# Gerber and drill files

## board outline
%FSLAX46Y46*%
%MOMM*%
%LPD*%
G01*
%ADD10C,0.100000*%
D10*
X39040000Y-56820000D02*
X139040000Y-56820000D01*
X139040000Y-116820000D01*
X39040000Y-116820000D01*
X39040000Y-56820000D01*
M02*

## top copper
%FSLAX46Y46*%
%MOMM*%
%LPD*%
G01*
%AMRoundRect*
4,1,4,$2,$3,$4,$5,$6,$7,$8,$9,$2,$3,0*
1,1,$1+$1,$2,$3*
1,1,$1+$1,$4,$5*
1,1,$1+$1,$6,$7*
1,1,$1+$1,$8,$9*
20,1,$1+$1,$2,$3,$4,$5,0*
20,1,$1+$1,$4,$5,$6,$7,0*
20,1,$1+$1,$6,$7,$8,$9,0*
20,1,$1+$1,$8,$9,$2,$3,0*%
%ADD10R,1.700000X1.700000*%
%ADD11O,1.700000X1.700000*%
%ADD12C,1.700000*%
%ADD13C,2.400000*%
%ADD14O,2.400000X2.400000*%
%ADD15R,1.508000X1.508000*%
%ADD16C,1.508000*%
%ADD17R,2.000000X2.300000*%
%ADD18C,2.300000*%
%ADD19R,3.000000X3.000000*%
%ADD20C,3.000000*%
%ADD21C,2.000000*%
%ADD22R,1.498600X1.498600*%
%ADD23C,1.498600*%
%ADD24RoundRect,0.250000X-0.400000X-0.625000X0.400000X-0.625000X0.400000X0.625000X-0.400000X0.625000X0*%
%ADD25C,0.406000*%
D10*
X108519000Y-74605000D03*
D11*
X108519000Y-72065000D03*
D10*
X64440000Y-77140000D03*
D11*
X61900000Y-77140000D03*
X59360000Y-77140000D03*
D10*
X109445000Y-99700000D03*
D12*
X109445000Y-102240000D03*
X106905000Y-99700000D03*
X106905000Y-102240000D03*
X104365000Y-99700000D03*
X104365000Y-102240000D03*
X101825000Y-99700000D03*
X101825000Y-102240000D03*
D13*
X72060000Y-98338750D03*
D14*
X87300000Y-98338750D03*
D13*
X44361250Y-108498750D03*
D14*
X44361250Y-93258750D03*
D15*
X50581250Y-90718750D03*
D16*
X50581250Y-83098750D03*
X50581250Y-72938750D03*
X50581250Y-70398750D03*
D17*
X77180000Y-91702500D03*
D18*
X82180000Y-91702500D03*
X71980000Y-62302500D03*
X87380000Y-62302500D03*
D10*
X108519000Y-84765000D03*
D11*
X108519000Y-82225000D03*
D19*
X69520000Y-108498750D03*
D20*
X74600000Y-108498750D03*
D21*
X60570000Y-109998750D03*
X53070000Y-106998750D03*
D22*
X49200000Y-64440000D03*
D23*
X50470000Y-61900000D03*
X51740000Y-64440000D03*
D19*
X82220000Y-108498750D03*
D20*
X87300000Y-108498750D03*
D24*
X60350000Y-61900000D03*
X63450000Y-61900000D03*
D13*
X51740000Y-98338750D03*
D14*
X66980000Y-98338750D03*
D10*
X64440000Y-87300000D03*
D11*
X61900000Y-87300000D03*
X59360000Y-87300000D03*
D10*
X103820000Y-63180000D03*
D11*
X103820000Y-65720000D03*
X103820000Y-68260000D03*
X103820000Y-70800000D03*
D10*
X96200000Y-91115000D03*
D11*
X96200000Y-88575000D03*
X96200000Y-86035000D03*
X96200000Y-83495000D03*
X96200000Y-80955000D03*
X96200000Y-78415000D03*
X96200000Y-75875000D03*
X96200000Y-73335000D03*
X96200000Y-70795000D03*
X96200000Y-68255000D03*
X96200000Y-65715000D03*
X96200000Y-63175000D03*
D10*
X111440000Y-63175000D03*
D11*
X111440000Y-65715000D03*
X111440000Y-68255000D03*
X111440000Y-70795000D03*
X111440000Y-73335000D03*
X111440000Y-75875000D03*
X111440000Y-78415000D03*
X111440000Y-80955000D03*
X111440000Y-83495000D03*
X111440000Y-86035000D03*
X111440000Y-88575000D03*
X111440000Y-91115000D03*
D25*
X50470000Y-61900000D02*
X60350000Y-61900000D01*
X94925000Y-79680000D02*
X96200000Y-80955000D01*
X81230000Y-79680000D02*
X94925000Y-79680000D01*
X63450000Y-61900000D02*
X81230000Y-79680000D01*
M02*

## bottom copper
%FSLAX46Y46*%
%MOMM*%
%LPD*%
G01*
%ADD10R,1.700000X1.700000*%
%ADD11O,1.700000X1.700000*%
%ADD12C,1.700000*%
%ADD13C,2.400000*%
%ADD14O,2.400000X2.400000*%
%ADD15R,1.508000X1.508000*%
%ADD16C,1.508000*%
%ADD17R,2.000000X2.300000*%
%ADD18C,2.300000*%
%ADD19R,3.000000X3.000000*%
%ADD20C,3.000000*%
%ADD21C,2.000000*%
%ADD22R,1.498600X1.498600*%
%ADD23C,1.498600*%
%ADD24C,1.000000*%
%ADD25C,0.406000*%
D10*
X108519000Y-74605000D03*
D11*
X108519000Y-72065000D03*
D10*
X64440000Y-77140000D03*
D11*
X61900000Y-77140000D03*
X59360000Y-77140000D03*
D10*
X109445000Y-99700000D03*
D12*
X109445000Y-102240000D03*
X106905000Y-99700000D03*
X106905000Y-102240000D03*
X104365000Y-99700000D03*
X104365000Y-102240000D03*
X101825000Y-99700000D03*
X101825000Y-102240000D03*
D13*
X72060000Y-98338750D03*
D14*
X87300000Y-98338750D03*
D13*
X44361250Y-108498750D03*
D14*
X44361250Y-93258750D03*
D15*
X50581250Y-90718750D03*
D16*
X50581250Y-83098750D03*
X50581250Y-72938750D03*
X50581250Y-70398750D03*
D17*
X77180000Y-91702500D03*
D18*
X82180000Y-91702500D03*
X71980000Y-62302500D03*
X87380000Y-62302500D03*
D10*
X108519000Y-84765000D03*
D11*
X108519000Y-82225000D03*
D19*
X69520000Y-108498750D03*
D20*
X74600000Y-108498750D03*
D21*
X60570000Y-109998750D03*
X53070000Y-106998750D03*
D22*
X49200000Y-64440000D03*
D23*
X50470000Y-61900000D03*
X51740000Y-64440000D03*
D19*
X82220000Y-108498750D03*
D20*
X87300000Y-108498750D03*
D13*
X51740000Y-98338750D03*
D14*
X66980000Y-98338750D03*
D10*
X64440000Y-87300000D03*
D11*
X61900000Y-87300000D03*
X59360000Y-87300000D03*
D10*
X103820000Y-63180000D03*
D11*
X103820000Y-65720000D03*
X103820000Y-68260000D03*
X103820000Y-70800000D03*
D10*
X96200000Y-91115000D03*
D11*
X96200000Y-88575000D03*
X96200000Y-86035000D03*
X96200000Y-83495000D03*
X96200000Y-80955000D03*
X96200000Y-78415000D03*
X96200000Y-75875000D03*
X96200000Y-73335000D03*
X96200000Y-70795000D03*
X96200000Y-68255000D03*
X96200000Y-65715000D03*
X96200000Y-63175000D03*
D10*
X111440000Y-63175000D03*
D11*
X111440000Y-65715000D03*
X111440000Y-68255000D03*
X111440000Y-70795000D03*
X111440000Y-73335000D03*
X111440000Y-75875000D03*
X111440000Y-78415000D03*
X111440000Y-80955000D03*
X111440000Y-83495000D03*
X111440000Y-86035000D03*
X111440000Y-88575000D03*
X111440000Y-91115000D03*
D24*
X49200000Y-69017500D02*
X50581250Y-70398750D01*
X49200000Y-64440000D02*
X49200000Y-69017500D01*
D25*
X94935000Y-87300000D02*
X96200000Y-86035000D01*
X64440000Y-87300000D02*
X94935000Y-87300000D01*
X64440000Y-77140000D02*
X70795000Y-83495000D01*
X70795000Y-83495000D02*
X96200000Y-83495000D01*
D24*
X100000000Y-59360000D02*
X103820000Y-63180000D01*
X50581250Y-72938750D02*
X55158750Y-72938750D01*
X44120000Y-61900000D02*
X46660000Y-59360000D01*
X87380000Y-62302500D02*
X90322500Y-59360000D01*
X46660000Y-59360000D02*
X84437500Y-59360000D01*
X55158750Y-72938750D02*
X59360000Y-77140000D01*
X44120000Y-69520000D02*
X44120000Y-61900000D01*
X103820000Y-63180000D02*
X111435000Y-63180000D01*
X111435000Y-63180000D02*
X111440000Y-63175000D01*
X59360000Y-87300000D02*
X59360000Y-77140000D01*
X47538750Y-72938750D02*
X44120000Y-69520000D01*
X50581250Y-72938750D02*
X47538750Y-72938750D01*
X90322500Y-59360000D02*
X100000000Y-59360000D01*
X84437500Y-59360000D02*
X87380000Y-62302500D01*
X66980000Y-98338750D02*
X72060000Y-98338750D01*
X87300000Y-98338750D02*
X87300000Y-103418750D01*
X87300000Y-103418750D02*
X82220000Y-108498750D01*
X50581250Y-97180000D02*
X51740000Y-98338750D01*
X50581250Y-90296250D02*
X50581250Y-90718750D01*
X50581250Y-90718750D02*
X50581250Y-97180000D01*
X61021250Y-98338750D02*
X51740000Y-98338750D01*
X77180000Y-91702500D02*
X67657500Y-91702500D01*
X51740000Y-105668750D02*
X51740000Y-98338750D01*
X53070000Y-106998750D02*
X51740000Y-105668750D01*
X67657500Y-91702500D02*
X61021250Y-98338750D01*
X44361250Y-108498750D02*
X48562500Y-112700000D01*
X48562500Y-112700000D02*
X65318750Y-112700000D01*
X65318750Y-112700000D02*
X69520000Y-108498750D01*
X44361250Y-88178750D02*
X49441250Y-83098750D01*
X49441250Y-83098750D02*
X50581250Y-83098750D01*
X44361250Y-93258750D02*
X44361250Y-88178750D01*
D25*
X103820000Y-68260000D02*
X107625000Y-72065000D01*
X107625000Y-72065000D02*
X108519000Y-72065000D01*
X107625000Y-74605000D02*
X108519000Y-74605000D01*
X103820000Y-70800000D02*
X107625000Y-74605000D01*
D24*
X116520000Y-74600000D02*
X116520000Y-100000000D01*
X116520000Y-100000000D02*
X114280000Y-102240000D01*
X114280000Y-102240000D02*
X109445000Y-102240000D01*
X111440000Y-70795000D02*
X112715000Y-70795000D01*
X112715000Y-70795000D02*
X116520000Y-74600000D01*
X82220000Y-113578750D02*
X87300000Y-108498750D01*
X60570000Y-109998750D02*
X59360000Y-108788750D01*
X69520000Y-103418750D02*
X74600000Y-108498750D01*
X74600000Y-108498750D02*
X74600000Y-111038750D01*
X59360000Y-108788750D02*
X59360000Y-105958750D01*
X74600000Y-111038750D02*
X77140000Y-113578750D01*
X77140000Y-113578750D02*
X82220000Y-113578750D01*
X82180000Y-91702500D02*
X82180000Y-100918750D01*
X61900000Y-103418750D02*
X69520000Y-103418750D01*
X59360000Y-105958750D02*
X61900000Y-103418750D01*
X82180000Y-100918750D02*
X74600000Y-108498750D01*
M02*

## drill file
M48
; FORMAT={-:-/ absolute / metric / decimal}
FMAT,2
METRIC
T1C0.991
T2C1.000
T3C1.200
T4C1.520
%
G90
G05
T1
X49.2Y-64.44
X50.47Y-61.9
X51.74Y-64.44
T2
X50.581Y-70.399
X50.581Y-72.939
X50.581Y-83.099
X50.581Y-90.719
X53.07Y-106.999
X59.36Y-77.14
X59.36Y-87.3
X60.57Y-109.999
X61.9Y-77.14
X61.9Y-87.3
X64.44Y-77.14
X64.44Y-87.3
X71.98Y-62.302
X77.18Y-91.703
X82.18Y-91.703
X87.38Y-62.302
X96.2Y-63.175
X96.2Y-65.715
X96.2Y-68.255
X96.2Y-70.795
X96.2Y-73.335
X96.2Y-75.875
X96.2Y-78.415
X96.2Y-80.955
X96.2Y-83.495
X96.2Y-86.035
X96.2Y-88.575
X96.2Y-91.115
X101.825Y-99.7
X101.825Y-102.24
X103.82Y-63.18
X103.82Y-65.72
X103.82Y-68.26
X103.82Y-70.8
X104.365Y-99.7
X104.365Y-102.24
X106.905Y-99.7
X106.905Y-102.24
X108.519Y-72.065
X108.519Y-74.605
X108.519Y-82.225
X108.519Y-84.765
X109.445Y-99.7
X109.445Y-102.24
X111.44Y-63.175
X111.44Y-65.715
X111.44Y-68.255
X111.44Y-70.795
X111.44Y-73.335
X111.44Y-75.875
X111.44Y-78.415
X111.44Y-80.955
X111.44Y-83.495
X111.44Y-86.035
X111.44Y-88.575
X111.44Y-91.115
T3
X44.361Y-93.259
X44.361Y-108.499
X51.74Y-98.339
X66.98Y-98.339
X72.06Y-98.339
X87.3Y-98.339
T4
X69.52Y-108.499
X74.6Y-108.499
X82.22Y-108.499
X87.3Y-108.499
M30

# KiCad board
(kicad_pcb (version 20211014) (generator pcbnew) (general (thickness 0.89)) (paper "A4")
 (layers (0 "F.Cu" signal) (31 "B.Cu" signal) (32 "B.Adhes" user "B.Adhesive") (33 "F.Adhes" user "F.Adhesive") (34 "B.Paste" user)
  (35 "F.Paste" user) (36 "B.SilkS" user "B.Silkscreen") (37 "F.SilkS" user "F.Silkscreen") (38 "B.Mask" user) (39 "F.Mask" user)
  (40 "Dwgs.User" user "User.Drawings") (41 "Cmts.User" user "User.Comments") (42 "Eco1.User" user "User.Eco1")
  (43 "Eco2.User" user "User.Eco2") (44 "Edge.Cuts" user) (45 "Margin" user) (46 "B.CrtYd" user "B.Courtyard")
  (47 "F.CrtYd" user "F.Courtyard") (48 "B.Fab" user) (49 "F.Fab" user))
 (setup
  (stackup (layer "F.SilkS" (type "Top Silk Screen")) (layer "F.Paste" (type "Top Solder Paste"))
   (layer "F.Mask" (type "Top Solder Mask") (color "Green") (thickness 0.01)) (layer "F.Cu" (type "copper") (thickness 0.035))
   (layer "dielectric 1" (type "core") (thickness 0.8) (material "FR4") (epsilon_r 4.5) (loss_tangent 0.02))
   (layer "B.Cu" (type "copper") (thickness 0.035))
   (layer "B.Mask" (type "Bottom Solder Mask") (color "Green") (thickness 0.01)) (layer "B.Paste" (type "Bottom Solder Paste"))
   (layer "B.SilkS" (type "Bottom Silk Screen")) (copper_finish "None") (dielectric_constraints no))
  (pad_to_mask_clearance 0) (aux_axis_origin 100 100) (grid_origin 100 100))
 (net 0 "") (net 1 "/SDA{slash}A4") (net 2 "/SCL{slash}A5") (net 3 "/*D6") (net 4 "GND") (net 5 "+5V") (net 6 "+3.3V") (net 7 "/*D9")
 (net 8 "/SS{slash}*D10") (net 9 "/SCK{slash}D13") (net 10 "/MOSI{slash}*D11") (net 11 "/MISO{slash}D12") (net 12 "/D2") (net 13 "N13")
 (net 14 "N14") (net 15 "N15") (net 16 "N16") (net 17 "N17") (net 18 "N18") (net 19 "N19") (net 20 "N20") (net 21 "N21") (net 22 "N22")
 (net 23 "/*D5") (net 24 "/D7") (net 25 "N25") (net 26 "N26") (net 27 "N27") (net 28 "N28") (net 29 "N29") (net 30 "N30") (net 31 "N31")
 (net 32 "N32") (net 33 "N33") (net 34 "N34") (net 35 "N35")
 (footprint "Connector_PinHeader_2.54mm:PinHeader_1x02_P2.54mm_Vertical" (layer "F.Cu") (at 108.519 74.605 180)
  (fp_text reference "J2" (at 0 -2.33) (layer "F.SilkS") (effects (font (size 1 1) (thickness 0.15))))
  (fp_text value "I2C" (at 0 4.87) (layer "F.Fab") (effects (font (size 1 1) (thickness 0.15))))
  (pad "1" thru_hole rect locked (at 0 0 180) (size 1.7 1.7) (drill 1) (layers *.Cu *.Mask) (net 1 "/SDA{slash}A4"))
  (pad "2" thru_hole oval locked (at 0 2.54 180) (size 1.7 1.7) (drill 1) (layers *.Cu *.Mask) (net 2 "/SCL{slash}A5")))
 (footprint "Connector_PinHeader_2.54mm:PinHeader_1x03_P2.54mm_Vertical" (layer "F.Cu") (at 64.44 77.14 -90)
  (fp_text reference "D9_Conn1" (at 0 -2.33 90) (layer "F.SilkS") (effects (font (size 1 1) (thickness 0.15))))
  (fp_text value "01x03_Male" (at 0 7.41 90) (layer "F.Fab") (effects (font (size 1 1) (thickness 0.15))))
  (pad "1" thru_hole rect (at 0 0 270) (size 1.7 1.7) (drill 1) (layers *.Cu *.Mask) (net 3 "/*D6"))
  (pad "2" thru_hole oval (at 0 2.54 270) (size 1.7 1.7) (drill 1) (layers *.Cu *.Mask) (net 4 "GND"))
  (pad "3" thru_hole oval (at 0 5.08 270) (size 1.7 1.7) (drill 1) (layers *.Cu *.Mask) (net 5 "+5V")))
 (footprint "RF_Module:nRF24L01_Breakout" (layer "F.Cu") (at 109.445 99.7 -90)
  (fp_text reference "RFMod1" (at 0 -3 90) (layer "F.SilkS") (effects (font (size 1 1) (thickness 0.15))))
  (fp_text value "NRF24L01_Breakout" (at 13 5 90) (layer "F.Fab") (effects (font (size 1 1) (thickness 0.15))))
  (pad "1" thru_hole rect (at 0 0 270) (size 1.7 1.7) (drill 1) (layers *.Cu *.Mask) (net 4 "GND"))
  (pad "2" thru_hole circle (at 2.54 0 270) (size 1.7 1.7) (drill 1) (layers *.Cu *.Mask) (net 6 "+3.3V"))
  (pad "3" thru_hole circle (at 0 2.54 270) (size 1.7 1.7) (drill 1) (layers *.Cu *.Mask) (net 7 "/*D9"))
  (pad "4" thru_hole circle (at 2.54 2.54 270) (size 1.7 1.7) (drill 1) (layers *.Cu *.Mask) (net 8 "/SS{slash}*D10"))
  (pad "5" thru_hole circle (at 0 5.08 270) (size 1.7 1.7) (drill 1) (layers *.Cu *.Mask) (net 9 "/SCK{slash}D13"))
  (pad "6" thru_hole circle (at 2.54 5.08 270) (size 1.7 1.7) (drill 1) (layers *.Cu *.Mask) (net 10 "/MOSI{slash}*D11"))
  (pad "7" thru_hole circle (at 0 7.62 270) (size 1.7 1.7) (drill 1) (layers *.Cu *.Mask) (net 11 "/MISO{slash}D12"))
  (pad "8" thru_hole circle (at 2.54 7.62 270) (size 1.7 1.7) (drill 1) (layers *.Cu *.Mask) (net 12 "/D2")))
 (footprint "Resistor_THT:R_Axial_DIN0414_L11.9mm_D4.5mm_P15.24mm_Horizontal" (layer "F.Cu") (at 72.06 98.33875)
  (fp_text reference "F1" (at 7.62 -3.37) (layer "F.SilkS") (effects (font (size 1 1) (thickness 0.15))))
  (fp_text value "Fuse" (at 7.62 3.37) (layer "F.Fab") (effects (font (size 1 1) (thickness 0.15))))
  (pad "1" thru_hole circle (at 0 0) (size 2.4 2.4) (drill 1.2) (layers *.Cu *.Mask) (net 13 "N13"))
  (pad "2" thru_hole oval (at 15.24 0) (size 2.4 2.4) (drill 1.2) (layers *.Cu *.Mask) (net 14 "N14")))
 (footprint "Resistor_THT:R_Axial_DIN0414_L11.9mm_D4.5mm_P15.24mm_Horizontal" (layer "F.Cu") (at 44.36125 108.49875 90)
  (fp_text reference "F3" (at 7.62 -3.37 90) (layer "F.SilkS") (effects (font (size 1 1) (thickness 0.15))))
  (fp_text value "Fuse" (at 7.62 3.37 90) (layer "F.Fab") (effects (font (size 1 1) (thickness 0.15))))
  (pad "1" thru_hole circle (at 0 0 90) (size 2.4 2.4) (drill 1.2) (layers *.Cu *.Mask) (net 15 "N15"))
  (pad "2" thru_hole oval (at 15.24 0 90) (size 2.4 2.4) (drill 1.2) (layers *.Cu *.Mask) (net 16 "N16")))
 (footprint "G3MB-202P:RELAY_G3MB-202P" (layer "F.Cu") (at 51.98125 80.55875 -90)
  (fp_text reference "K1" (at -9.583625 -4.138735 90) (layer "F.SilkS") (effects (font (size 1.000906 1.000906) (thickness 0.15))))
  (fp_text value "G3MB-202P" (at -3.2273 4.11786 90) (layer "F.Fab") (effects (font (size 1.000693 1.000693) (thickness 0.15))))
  (pad "1" thru_hole rect locked (at 10.16 1.4 270) (size 1.508 1.508) (drill 1) (layers *.Cu *.Mask) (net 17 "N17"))
  (pad "2" thru_hole circle locked (at 2.54 1.4 270) (size 1.508 1.508) (drill 1) (layers *.Cu *.Mask) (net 16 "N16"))
  (pad "3" thru_hole circle locked (at -7.62 1.4 270) (size 1.508 1.508) (drill 1) (layers *.Cu *.Mask) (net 5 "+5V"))
  (pad "4" thru_hole circle locked (at -10.16 1.4 270) (size 1.508 1.508) (drill 1) (layers *.Cu *.Mask) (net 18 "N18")))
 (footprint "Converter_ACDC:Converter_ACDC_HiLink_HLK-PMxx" (layer "F.Cu") (at 77.18 91.7025 90)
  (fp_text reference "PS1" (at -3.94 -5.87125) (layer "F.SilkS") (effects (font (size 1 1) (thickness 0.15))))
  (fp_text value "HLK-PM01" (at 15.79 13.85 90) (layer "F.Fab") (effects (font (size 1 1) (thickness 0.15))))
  (pad "1" thru_hole rect (at 0 0 90) (size 2.3 2) (drill 1) (layers *.Cu *.Mask) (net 17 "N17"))
  (pad "2" thru_hole circle (at 0 5 90) (size 2.3 2.3) (drill 1) (layers *.Cu *.Mask) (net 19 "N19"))
  (pad "3" thru_hole circle (at 29.4 -5.2 90) (size 2.3 2.3) (drill 1) (layers *.Cu *.Mask) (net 4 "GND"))
  (pad "4" thru_hole circle (at 29.4 10.2 90) (size 2.3 2.3) (drill 1) (layers *.Cu *.Mask) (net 5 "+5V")))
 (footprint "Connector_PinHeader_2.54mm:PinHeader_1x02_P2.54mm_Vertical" (layer "F.Cu") (at 108.519 84.765 180)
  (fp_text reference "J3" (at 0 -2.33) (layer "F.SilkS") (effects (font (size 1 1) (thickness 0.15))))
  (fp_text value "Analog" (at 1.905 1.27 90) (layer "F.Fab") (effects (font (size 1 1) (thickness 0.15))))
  (pad "1" thru_hole rect locked (at 0 0 180) (size 1.7 1.7) (drill 1) (layers *.Cu *.Mask) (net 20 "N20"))
  (pad "2" thru_hole oval locked (at 0 2.54 180) (size 1.7 1.7) (drill 1) (layers *.Cu *.Mask) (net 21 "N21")))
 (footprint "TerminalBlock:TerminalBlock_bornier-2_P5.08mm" (layer "F.Cu") (at 69.52 108.49875)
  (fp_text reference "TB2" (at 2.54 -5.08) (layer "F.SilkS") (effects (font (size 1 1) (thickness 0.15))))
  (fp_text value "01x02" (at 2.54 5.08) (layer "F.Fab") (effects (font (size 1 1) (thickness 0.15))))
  (pad "1" thru_hole rect (at 0 0) (size 3 3) (drill 1.52) (layers *.Cu *.Mask) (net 15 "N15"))
  (pad "2" thru_hole circle (at 5.08 0) (size 3 3) (drill 1.52) (layers *.Cu *.Mask) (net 19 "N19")))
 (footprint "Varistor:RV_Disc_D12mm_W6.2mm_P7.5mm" (layer "F.Cu") (at 60.57 109.99875 180)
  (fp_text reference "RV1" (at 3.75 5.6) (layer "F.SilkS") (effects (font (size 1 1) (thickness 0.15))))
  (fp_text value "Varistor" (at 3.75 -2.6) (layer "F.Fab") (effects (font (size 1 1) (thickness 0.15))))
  (pad "1" thru_hole circle (at 0 0 180) (size 2 2) (drill 1) (layers *.Cu *.Mask) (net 19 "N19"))
  (pad "2" thru_hole circle (at 7.5 3 180) (size 2 2) (drill 1) (layers *.Cu *.Mask) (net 17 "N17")))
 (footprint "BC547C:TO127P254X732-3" (layer "F.Cu") (at 51.74 61.9)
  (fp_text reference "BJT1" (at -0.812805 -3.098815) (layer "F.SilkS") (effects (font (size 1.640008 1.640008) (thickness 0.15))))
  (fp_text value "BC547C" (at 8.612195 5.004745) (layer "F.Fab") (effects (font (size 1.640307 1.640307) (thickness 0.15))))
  (pad "1" thru_hole rect locked (at -2.54 2.54) (size 1.4986 1.4986) (drill 0.9906) (layers *.Cu *.Mask) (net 18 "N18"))
  (pad "2" thru_hole circle locked (at -1.27 0) (size 1.4986 1.4986) (drill 0.9906) (layers *.Cu *.Mask) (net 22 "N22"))
  (pad "3" thru_hole circle locked (at 0 2.54) (size 1.4986 1.4986) (drill 0.9906) (layers *.Cu *.Mask) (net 4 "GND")))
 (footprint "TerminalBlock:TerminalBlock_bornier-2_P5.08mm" (layer "F.Cu") (at 82.22 108.49875)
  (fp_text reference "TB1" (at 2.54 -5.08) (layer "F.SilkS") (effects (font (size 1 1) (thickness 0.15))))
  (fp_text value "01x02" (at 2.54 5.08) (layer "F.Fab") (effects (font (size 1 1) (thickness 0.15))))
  (pad "1" thru_hole rect (at 0 0) (size 3 3) (drill 1.52) (layers *.Cu *.Mask) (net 14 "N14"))
  (pad "2" thru_hole circle (at 5.08 0) (size 3 3) (drill 1.52) (layers *.Cu *.Mask) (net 19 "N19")))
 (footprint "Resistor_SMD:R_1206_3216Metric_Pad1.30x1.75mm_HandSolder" (layer "F.Cu") (at 61.9 61.9)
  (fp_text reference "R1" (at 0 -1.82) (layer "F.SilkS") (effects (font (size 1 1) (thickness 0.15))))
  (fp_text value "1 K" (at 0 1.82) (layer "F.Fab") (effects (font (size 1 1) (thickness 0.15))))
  (pad "1" smd roundrect (at -1.55 0) (size 1.3 1.75) (layers "F.Cu" "F.Paste" "F.Mask") (roundrect_rratio 0.192308) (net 22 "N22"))
  (pad "2" smd roundrect (at 1.55 0) (size 1.3 1.75) (layers "F.Cu" "F.Paste" "F.Mask") (roundrect_rratio 0.192308) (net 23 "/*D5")))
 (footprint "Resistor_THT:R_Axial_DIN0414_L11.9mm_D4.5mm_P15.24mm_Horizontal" (layer "F.Cu") (at 51.74 98.33875)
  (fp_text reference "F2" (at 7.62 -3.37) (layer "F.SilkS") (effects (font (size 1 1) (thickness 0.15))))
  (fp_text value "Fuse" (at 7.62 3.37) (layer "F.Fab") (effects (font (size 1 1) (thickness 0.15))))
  (pad "1" thru_hole circle (at 0 0) (size 2.4 2.4) (drill 1.2) (layers *.Cu *.Mask) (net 17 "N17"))
  (pad "2" thru_hole oval (at 15.24 0) (size 2.4 2.4) (drill 1.2) (layers *.Cu *.Mask) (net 13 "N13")))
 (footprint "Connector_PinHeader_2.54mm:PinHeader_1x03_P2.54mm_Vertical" (layer "F.Cu") (at 64.44 87.3 -90)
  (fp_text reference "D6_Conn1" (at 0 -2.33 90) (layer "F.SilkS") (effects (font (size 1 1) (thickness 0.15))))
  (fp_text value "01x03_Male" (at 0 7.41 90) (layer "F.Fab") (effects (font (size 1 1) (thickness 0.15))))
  (pad "1" thru_hole rect (at 0 0 270) (size 1.7 1.7) (drill 1) (layers *.Cu *.Mask) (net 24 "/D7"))
  (pad "2" thru_hole oval (at 0 2.54 270) (size 1.7 1.7) (drill 1) (layers *.Cu *.Mask) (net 4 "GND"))
  (pad "3" thru_hole oval (at 0 5.08 270) (size 1.7 1.7) (drill 1) (layers *.Cu *.Mask) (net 5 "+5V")))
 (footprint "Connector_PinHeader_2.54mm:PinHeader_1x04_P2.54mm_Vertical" (layer "F.Cu") (at 103.82 63.18)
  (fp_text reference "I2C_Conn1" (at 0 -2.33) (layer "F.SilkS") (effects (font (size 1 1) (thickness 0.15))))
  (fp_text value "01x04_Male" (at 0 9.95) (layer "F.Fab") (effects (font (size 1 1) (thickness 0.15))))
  (pad "1" thru_hole rect (at 0 0) (size 1.7 1.7) (drill 1) (layers *.Cu *.Mask) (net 5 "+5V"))
  (pad "2" thru_hole oval (at 0 2.54) (size 1.7 1.7) (drill 1) (layers *.Cu *.Mask) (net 4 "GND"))
  (pad "3" thru_hole oval (at 0 5.08) (size 1.7 1.7) (drill 1) (layers *.Cu *.Mask) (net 2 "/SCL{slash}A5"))
  (pad "4" thru_hole oval (at 0 7.62) (size 1.7 1.7) (drill 1) (layers *.Cu *.Mask) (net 1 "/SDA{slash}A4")))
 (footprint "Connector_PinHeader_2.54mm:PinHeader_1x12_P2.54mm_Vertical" (layer "B.Cu") (at 96.2 91.115)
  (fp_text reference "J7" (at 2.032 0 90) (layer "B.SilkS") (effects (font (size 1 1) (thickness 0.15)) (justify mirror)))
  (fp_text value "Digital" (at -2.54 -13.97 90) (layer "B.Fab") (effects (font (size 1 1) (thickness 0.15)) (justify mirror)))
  (pad "1" thru_hole rect locked (at 0 0) (size 1.7 1.7) (drill 1) (layers *.Cu *.Mask) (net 7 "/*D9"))
  (pad "2" thru_hole oval locked (at 0 -2.54) (size 1.7 1.7) (drill 1) (layers *.Cu *.Mask) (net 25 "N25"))
  (pad "3" thru_hole oval locked (at 0 -5.08) (size 1.7 1.7) (drill 1) (layers *.Cu *.Mask) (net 24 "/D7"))
  (pad "4" thru_hole oval locked (at 0 -7.62) (size 1.7 1.7) (drill 1) (layers *.Cu *.Mask) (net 3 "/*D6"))
  (pad "5" thru_hole oval locked (at 0 -10.16) (size 1.7 1.7) (drill 1) (layers *.Cu *.Mask) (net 23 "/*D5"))
  (pad "6" thru_hole oval locked (at 0 -12.7) (size 1.7 1.7) (drill 1) (layers *.Cu *.Mask) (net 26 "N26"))
  (pad "7" thru_hole oval locked (at 0 -15.24) (size 1.7 1.7) (drill 1) (layers *.Cu *.Mask) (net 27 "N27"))
  (pad "8" thru_hole oval locked (at 0 -17.78) (size 1.7 1.7) (drill 1) (layers *.Cu *.Mask) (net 12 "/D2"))
  (pad "9" thru_hole oval locked (at 0 -20.32) (size 1.7 1.7) (drill 1) (layers *.Cu *.Mask) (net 4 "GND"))
  (pad "10" thru_hole oval locked (at 0 -22.86) (size 1.7 1.7) (drill 1) (layers *.Cu *.Mask) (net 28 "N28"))
  (pad "11" thru_hole oval locked (at 0 -25.4) (size 1.7 1.7) (drill 1) (layers *.Cu *.Mask) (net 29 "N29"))
  (pad "12" thru_hole oval locked (at 0 -27.94) (size 1.7 1.7) (drill 1) (layers *.Cu *.Mask) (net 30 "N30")))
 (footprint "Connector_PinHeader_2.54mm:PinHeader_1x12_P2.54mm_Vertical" (layer "B.Cu") (at 111.44 63.175 180)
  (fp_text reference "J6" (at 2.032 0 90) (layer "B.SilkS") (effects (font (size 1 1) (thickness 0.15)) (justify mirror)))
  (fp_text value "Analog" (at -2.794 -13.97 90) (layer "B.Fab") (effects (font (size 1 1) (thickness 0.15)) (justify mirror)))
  (pad "1" thru_hole rect locked (at 0 0 180) (size 1.7 1.7) (drill 1) (layers *.Cu *.Mask) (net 5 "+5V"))
  (pad "2" thru_hole oval locked (at 0 -2.54 180) (size 1.7 1.7) (drill 1) (layers *.Cu *.Mask) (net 4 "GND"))
  (pad "3" thru_hole oval locked (at 0 -5.08 180) (size 1.7 1.7) (drill 1) (layers *.Cu *.Mask) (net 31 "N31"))
  (pad "4" thru_hole oval locked (at 0 -7.62 180) (size 1.7 1.7) (drill 1) (layers *.Cu *.Mask) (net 6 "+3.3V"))
  (pad "5" thru_hole oval locked (at 0 -10.16 180) (size 1.7 1.7) (drill 1) (layers *.Cu *.Mask) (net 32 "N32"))
  (pad "6" thru_hole oval locked (at 0 -12.7 180) (size 1.7 1.7) (drill 1) (layers *.Cu *.Mask) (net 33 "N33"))
  (pad "7" thru_hole oval locked (at 0 -15.24 180) (size 1.7 1.7) (drill 1) (layers *.Cu *.Mask) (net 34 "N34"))
  (pad "8" thru_hole oval locked (at 0 -17.78 180) (size 1.7 1.7) (drill 1) (layers *.Cu *.Mask) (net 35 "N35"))
  (pad "9" thru_hole oval locked (at 0 -20.32 180) (size 1.7 1.7) (drill 1) (layers *.Cu *.Mask) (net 9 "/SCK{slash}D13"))
  (pad "10" thru_hole oval locked (at 0 -22.86 180) (size 1.7 1.7) (drill 1) (layers *.Cu *.Mask) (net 11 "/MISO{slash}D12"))
  (pad "11" thru_hole oval locked (at 0 -25.4 180) (size 1.7 1.7) (drill 1) (layers *.Cu *.Mask) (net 10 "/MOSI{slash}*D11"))
  (pad "12" thru_hole oval locked (at 0 -27.94 180) (size 1.7 1.7) (drill 1) (layers *.Cu *.Mask) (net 8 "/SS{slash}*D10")))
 (gr_rect (start 39.04 56.82) (end 139.04 116.82) (layer "Edge.Cuts") (width 0.1) (fill none))
 (segment (start 49.2 69.0175) (end 50.58125 70.39875) (width 1) (layer "B.Cu") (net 18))
 (segment (start 49.2 64.44) (end 49.2 69.0175) (width 1) (layer "B.Cu") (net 18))
 (segment (start 50.47 61.9) (end 60.35 61.9) (width 0.406) (layer "F.Cu") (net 22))
 (segment (start 94.935 87.3) (end 96.2 86.035) (width 0.406) (layer "B.Cu") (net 24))
 (segment (start 64.44 87.3) (end 94.935 87.3) (width 0.406) (layer "B.Cu") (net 24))
 (segment (start 64.44 77.14) (end 70.795 83.495) (width 0.406) (layer "B.Cu") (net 3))
 (segment (start 70.795 83.495) (end 96.2 83.495) (width 0.406) (layer "B.Cu") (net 3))
 (segment (start 94.925 79.68) (end 96.2 80.955) (width 0.406) (layer "F.Cu") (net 23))
 (segment (start 81.23 79.68) (end 94.925 79.68) (width 0.406) (layer "F.Cu") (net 23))
 (segment (start 63.45 61.9) (end 81.23 79.68) (width 0.406) (layer "F.Cu") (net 23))
 (segment (start 100 59.36) (end 103.82 63.18) (width 1) (layer "B.Cu") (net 5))
 (segment (start 50.58125 72.93875) (end 55.15875 72.93875) (width 1) (layer "B.Cu") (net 5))
 (segment (start 44.12 61.9) (end 46.66 59.36) (width 1) (layer "B.Cu") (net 5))
 (segment (start 87.38 62.3025) (end 90.3225 59.36) (width 1) (layer "B.Cu") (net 5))
 (segment (start 46.66 59.36) (end 84.4375 59.36) (width 1) (layer "B.Cu") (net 5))
 (segment (start 55.15875 72.93875) (end 59.36 77.14) (width 1) (layer "B.Cu") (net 5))
 (segment (start 44.12 69.52) (end 44.12 61.9) (width 1) (layer "B.Cu") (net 5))
 (segment (start 103.82 63.18) (end 111.435 63.18) (width 1) (layer "B.Cu") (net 5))
 (segment (start 111.435 63.18) (end 111.44 63.175) (width 1) (layer "B.Cu") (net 5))
 (segment (start 59.36 87.3) (end 59.36 77.14) (width 1) (layer "B.Cu") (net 5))
 (segment (start 47.53875 72.93875) (end 44.12 69.52) (width 1) (layer "B.Cu") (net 5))
 (segment (start 50.58125 72.93875) (end 47.53875 72.93875) (width 1) (layer "B.Cu") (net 5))
 (segment (start 90.3225 59.36) (end 100 59.36) (width 1) (layer "B.Cu") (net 5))
 (segment (start 84.4375 59.36) (end 87.38 62.3025) (width 1) (layer "B.Cu") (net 5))
 (segment (start 66.98 98.33875) (end 72.06 98.33875) (width 1) (layer "B.Cu") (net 13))
 (segment (start 87.3 98.33875) (end 87.3 103.41875) (width 1) (layer "B.Cu") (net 14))
 (segment (start 87.3 103.41875) (end 82.22 108.49875) (width 1) (layer "B.Cu") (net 14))
 (segment (start 50.58125 97.18) (end 51.74 98.33875) (width 1) (layer "B.Cu") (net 17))
 (segment (start 50.58125 90.29625) (end 50.58125 90.71875) (width 1) (layer "B.Cu") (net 17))
 (segment (start 50.58125 90.71875) (end 50.58125 97.18) (width 1) (layer "B.Cu") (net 17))
 (segment (start 61.02125 98.33875) (end 51.74 98.33875) (width 1) (layer "B.Cu") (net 17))
 (segment (start 77.18 91.7025) (end 67.6575 91.7025) (width 1) (layer "B.Cu") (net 17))
 (segment (start 51.74 105.66875) (end 51.74 98.33875) (width 1) (layer "B.Cu") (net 17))
 (segment (start 53.07 106.99875) (end 51.74 105.66875) (width 1) (layer "B.Cu") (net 17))
 (segment (start 67.6575 91.7025) (end 61.02125 98.33875) (width 1) (layer "B.Cu") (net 17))
 (segment (start 44.36125 108.49875) (end 48.5625 112.7) (width 1) (layer "B.Cu") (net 15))
 (segment (start 48.5625 112.7) (end 65.31875 112.7) (width 1) (layer "B.Cu") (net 15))
 (segment (start 65.31875 112.7) (end 69.52 108.49875) (width 1) (layer "B.Cu") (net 15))
 (segment (start 44.36125 88.17875) (end 49.44125 83.09875) (width 1) (layer "B.Cu") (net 16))
 (segment (start 49.44125 83.09875) (end 50.58125 83.09875) (width 1) (layer "B.Cu") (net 16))
 (segment (start 44.36125 93.25875) (end 44.36125 88.17875) (width 1) (layer "B.Cu") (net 16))
 (segment (start 103.82 68.26) (end 107.625 72.065) (width 0.406) (layer "B.Cu") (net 2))
 (segment (start 107.625 72.065) (end 108.519 72.065) (width 0.406) (layer "B.Cu") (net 2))
 (segment (start 107.625 74.605) (end 108.519 74.605) (width 0.406) (layer "B.Cu") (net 1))
 (segment (start 103.82 70.8) (end 107.625 74.605) (width 0.406) (layer "B.Cu") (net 1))
 (segment (start 116.52 74.6) (end 116.52 100) (width 1) (layer "B.Cu") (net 6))
 (segment (start 116.52 100) (end 114.28 102.24) (width 1) (layer "B.Cu") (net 6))
 (segment (start 114.28 102.24) (end 109.445 102.24) (width 1) (layer "B.Cu") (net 6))
 (segment (start 111.44 70.795) (end 112.715 70.795) (width 1) (layer "B.Cu") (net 6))
 (segment (start 112.715 70.795) (end 116.52 74.6) (width 1) (layer "B.Cu") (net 6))
 (segment (start 82.22 113.57875) (end 87.3 108.49875) (width 1) (layer "B.Cu") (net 19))
 (segment (start 60.57 109.99875) (end 59.36 108.78875) (width 1) (layer "B.Cu") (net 19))
 (segment (start 69.52 103.41875) (end 74.6 108.49875) (width 1) (layer "B.Cu") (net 19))
 (segment (start 74.6 108.49875) (end 74.6 111.03875) (width 1) (layer "B.Cu") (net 19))
 (segment (start 59.36 108.78875) (end 59.36 105.95875) (width 1) (layer "B.Cu") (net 19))
 (segment (start 74.6 111.03875) (end 77.14 113.57875) (width 1) (layer "B.Cu") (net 19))
 (segment (start 77.14 113.57875) (end 82.22 113.57875) (width 1) (layer "B.Cu") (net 19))
 (segment (start 82.18 91.7025) (end 82.18 100.91875) (width 1) (layer "B.Cu") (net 19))
 (segment (start 61.9 103.41875) (end 69.52 103.41875) (width 1) (layer "B.Cu") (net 19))
 (segment (start 59.36 105.95875) (end 61.9 103.41875) (width 1) (layer "B.Cu") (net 19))
 (segment (start 82.18 100.91875) (end 74.6 108.49875) (width 1) (layer "B.Cu") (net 19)))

